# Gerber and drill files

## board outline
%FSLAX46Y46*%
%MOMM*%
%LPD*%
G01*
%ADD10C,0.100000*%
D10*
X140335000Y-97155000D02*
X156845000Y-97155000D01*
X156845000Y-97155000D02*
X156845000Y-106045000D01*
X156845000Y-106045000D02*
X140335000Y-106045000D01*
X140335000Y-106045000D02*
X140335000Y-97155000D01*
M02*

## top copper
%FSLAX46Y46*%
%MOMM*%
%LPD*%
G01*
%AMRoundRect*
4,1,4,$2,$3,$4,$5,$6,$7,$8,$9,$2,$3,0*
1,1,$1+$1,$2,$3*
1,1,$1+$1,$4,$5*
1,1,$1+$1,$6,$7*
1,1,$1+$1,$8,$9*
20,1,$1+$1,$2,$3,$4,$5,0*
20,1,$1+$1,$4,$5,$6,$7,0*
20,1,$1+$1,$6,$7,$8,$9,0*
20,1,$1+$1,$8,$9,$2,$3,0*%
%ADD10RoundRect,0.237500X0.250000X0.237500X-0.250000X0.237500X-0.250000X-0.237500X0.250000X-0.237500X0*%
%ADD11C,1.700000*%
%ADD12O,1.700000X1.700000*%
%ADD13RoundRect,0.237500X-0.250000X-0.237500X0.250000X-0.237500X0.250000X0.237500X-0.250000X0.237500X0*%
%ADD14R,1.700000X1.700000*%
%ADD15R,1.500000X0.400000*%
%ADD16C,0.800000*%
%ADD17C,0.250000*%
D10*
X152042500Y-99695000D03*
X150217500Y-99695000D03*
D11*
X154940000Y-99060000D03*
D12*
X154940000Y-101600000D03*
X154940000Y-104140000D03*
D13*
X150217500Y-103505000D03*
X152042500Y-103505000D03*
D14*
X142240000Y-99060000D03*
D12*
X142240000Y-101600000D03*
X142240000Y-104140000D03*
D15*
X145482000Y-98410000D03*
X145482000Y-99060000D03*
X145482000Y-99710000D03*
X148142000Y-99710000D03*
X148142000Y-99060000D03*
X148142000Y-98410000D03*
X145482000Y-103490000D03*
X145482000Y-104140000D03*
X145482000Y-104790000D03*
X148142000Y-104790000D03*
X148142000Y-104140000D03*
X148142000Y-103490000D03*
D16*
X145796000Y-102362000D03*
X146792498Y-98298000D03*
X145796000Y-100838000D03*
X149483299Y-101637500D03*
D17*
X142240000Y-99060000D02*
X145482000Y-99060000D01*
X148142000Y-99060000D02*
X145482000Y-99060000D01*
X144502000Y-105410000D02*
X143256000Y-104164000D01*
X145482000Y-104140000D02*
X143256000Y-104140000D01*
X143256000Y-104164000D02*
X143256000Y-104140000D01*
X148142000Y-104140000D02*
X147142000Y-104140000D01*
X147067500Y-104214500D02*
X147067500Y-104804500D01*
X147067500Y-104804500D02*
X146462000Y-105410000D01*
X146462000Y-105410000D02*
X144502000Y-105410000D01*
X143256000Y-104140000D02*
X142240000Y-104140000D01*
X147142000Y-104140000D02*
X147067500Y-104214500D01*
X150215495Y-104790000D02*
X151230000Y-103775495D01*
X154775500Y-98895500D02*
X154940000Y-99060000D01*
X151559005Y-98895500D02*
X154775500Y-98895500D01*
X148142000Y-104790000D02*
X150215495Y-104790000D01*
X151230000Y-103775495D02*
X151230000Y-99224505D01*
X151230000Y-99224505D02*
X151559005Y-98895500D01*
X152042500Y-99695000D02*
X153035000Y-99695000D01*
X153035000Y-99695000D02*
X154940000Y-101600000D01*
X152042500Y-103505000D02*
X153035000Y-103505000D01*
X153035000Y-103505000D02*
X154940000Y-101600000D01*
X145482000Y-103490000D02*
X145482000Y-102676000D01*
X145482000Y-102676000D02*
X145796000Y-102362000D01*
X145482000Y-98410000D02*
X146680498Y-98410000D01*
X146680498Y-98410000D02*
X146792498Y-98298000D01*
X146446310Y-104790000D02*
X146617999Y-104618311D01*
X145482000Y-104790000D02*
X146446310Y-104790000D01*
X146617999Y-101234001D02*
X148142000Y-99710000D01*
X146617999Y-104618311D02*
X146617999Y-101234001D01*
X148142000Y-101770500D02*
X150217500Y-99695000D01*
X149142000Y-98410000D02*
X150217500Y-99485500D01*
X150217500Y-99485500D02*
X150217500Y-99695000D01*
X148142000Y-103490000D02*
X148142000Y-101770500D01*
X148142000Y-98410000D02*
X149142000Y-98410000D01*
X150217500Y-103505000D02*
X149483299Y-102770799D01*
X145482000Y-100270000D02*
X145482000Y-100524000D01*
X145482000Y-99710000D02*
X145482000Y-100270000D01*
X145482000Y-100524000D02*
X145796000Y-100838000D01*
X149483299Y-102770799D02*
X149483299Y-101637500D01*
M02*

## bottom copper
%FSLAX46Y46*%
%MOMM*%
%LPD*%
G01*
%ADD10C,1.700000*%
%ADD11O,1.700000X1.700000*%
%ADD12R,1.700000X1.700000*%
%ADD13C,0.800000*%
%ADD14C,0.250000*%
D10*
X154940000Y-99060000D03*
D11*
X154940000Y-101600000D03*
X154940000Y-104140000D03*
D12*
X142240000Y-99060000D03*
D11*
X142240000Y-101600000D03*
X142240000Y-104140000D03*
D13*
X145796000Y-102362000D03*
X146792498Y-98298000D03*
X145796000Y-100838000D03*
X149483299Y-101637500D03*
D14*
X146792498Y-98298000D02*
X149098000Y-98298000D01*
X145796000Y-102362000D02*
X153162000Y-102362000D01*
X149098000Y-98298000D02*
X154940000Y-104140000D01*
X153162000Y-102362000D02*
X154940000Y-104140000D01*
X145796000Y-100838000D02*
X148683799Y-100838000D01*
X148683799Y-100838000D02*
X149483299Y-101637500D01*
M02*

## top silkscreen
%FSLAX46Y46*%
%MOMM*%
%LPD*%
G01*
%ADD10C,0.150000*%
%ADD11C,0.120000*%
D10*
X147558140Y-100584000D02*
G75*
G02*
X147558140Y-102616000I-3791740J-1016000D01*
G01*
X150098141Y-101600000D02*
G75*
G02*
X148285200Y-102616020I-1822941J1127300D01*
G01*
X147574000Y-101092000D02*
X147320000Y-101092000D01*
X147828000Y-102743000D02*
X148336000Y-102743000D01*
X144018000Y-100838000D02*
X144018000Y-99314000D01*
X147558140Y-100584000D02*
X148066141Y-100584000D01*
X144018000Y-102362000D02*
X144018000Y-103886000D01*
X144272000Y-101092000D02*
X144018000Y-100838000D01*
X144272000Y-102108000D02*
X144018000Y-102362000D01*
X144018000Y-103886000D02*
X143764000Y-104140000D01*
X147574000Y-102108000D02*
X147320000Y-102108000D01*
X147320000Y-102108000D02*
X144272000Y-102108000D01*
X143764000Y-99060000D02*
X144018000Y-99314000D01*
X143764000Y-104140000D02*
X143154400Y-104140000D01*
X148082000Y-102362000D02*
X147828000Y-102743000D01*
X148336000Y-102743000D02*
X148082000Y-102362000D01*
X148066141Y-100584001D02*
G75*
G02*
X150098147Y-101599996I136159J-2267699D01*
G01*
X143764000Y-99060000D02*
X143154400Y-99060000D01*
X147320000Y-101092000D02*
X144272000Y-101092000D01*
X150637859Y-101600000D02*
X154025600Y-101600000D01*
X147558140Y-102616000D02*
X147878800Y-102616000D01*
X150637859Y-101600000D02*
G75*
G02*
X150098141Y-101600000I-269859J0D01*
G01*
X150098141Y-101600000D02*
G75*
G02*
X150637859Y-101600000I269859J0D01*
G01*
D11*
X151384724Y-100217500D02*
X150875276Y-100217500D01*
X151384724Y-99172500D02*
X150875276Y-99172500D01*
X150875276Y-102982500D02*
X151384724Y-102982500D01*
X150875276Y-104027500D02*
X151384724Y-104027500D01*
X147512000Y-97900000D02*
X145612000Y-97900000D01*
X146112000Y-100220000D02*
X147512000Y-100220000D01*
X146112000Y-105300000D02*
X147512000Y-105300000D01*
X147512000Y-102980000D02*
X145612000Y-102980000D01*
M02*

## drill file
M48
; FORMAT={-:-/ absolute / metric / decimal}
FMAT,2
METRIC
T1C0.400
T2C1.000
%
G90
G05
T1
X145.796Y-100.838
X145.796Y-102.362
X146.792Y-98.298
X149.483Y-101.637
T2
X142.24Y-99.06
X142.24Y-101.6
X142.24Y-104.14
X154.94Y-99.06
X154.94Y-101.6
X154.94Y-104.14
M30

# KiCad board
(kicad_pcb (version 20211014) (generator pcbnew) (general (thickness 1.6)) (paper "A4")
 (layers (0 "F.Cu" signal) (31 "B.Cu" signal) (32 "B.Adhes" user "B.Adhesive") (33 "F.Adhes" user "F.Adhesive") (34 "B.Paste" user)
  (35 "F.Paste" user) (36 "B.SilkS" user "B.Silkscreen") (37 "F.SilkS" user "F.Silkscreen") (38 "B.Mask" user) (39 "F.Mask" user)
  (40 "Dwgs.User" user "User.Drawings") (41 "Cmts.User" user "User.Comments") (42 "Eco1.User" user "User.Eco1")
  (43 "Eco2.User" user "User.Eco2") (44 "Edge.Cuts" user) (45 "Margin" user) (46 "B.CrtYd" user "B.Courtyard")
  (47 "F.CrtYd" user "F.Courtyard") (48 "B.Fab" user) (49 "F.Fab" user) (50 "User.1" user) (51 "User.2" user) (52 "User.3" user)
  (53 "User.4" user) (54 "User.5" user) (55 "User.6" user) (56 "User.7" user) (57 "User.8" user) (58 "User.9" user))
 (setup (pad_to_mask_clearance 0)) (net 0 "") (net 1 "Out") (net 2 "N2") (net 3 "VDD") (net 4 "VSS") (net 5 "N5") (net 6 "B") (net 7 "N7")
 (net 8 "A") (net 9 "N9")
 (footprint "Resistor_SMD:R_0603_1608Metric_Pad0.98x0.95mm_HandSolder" (layer "F.Cu") (at 151.13 99.695 180)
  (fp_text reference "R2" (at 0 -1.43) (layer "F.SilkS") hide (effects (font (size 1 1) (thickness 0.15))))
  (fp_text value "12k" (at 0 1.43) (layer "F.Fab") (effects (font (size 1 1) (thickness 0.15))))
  (fp_line (start -0.254724 -0.5225) (end 0.254724 -0.5225) (layer "F.SilkS") (width 0.12))
  (fp_line (start -0.254724 0.5225) (end 0.254724 0.5225) (layer "F.SilkS") (width 0.12))
  (pad "1" smd roundrect (at -0.9125 0 180) (size 0.975 0.95) (layers "F.Cu" "F.Paste" "F.Mask") (roundrect_rratio 0.25) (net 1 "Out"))
  (pad "2" smd roundrect (at 0.9125 0 180) (size 0.975 0.95) (layers "F.Cu" "F.Paste" "F.Mask") (roundrect_rratio 0.25) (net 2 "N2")))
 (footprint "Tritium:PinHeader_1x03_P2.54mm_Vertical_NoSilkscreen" (layer "F.Cu") (at 154.94 99.06)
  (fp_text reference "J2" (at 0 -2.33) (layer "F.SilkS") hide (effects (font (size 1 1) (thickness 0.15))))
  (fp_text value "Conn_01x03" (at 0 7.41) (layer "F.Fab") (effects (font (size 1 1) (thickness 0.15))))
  (pad "1" thru_hole circle (at 0 0) (size 1.7 1.7) (drill 1) (layers *.Cu *.Mask) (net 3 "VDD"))
  (pad "2" thru_hole oval (at 0 2.54) (size 1.7 1.7) (drill 1) (layers *.Cu *.Mask) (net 1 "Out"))
  (pad "3" thru_hole oval (at 0 5.08) (size 1.7 1.7) (drill 1) (layers *.Cu *.Mask) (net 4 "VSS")))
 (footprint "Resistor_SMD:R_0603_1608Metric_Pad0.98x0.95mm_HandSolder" (layer "F.Cu") (at 151.13 103.505)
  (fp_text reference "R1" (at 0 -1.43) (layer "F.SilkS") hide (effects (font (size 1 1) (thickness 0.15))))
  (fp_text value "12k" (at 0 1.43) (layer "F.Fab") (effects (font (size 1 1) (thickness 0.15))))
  (fp_line (start -0.254724 -0.5225) (end 0.254724 -0.5225) (layer "F.SilkS") (width 0.12))
  (fp_line (start -0.254724 0.5225) (end 0.254724 0.5225) (layer "F.SilkS") (width 0.12))
  (pad "1" smd roundrect (at -0.9125 0) (size 0.975 0.95) (layers "F.Cu" "F.Paste" "F.Mask") (roundrect_rratio 0.25) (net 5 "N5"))
  (pad "2" smd roundrect (at 0.9125 0) (size 0.975 0.95) (layers "F.Cu" "F.Paste" "F.Mask") (roundrect_rratio 0.25) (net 1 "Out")))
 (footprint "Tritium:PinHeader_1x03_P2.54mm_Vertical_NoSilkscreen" (layer "F.Cu") (at 142.24 99.06)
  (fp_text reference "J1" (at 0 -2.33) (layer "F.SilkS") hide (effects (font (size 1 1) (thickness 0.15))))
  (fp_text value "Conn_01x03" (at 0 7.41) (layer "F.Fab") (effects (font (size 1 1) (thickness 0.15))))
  (pad "1" thru_hole rect (at 0 0) (size 1.7 1.7) (drill 1) (layers *.Cu *.Mask) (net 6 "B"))
  (pad "2" thru_hole oval (at 0 2.54) (size 1.7 1.7) (drill 1) (layers *.Cu *.Mask) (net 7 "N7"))
  (pad "3" thru_hole oval (at 0 5.08) (size 1.7 1.7) (drill 1) (layers *.Cu *.Mask) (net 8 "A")))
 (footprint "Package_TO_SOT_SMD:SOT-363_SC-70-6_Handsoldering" (layer "F.Cu") (at 146.812 99.06)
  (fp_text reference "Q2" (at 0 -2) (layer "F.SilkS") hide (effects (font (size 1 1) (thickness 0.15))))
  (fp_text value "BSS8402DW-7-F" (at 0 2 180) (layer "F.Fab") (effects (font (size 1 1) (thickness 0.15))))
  (fp_line (start 0.7 -1.16) (end -1.2 -1.16) (layer "F.SilkS") (width 0.12))
  (fp_line (start -0.7 1.16) (end 0.7 1.16) (layer "F.SilkS") (width 0.12))
  (pad "1" smd rect (at -1.33 -0.65) (size 1.5 0.4) (layers "F.Cu" "F.Paste" "F.Mask") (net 4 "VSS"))
  (pad "2" smd rect (at -1.33 0) (size 1.5 0.4) (layers "F.Cu" "F.Paste" "F.Mask") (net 6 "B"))
  (pad "3" smd rect (at -1.33 0.65) (size 1.5 0.4) (layers "F.Cu" "F.Paste" "F.Mask") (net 5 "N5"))
  (pad "4" smd rect (at 1.33 0.65) (size 1.5 0.4) (layers "F.Cu" "F.Paste" "F.Mask") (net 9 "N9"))
  (pad "5" smd rect (at 1.33 0) (size 1.5 0.4) (layers "F.Cu" "F.Paste" "F.Mask") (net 6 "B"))
  (pad "6" smd rect (at 1.33 -0.65) (size 1.5 0.4) (layers "F.Cu" "F.Paste" "F.Mask") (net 2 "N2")))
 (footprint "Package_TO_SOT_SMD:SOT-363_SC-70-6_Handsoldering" (layer "F.Cu") (at 146.812 104.14)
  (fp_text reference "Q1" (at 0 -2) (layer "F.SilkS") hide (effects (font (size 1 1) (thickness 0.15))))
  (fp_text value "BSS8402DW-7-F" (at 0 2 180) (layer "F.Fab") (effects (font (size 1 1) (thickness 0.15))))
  (fp_line (start -0.7 1.16) (end 0.7 1.16) (layer "F.SilkS") (width 0.12))
  (fp_line (start 0.7 -1.16) (end -1.2 -1.16) (layer "F.SilkS") (width 0.12))
  (pad "1" smd rect (at -1.33 -0.65) (size 1.5 0.4) (layers "F.Cu" "F.Paste" "F.Mask") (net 4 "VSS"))
  (pad "2" smd rect (at -1.33 0) (size 1.5 0.4) (layers "F.Cu" "F.Paste" "F.Mask") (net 8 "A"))
  (pad "3" smd rect (at -1.33 0.65) (size 1.5 0.4) (layers "F.Cu" "F.Paste" "F.Mask") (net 9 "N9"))
  (pad "4" smd rect (at 1.33 0.65) (size 1.5 0.4) (layers "F.Cu" "F.Paste" "F.Mask") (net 3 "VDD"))
  (pad "5" smd rect (at 1.33 0) (size 1.5 0.4) (layers "F.Cu" "F.Paste" "F.Mask") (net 8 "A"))
  (pad "6" smd rect (at 1.33 -0.65) (size 1.5 0.4) (layers "F.Cu" "F.Paste" "F.Mask") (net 2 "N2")))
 (gr_arc (start 147.55814 100.584) (mid 147.6919 101.6) (end 147.55814 102.616) (layer "F.SilkS") (width 0.15))
 (gr_arc (start 150.098141 101.6) (mid 149.323048 102.342429) (end 148.2852 102.616) (layer "F.SilkS") (width 0.15))
 (gr_line (start 147.574 101.092) (end 147.32 101.092) (layer "F.SilkS") (width 0.15))
 (gr_line (start 147.828 102.743) (end 148.336 102.743) (layer "F.SilkS") (width 0.15))
 (gr_line (start 144.018 100.838) (end 144.018 99.314) (layer "F.SilkS") (width 0.15))
 (gr_line (start 147.55814 100.584) (end 148.066141 100.584) (layer "F.SilkS") (width 0.15))
 (gr_line (start 144.018 102.362) (end 144.018 103.886) (layer "F.SilkS") (width 0.15))
 (gr_line (start 144.272 101.092) (end 144.018 100.838) (layer "F.SilkS") (width 0.15))
 (gr_line (start 144.272 102.108) (end 144.018 102.362) (layer "F.SilkS") (width 0.15))
 (gr_line (start 144.018 103.886) (end 143.764 104.14) (layer "F.SilkS") (width 0.15))
 (gr_line (start 147.574 102.108) (end 147.32 102.108) (layer "F.SilkS") (width 0.15))
 (gr_line (start 147.32 102.108) (end 144.272 102.108) (layer "F.SilkS") (width 0.15))
 (gr_line (start 143.764 99.06) (end 144.018 99.314) (layer "F.SilkS") (width 0.15))
 (gr_line (start 143.764 104.14) (end 143.1544 104.14) (layer "F.SilkS") (width 0.15))
 (gr_line (start 148.082 102.362) (end 147.828 102.743) (layer "F.SilkS") (width 0.15))
 (gr_line (start 148.336 102.743) (end 148.082 102.362) (layer "F.SilkS") (width 0.15))
 (gr_arc (start 148.066141 100.584001) (mid 149.218261 100.819761) (end 150.098141 101.6) (layer "F.SilkS") (width 0.15))
 (gr_line (start 143.764 99.06) (end 143.1544 99.06) (layer "F.SilkS") (width 0.15))
 (gr_line (start 147.32 101.092) (end 144.272 101.092) (layer "F.SilkS") (width 0.15))
 (gr_line (start 150.637859 101.6) (end 154.0256 101.6) (layer "F.SilkS") (width 0.15))
 (gr_line (start 147.55814 102.616) (end 147.8788 102.616) (layer "F.SilkS") (width 0.15))
 (gr_circle (center 150.368 101.6) (end 150.098141 101.6) (layer "F.SilkS") (width 0.15) (fill none))
 (gr_line (start 140.335 97.155) (end 156.845 97.155) (layer "Edge.Cuts") (width 0.1))
 (gr_line (start 156.845 97.155) (end 156.845 106.045) (layer "Edge.Cuts") (width 0.1))
 (gr_line (start 156.845 106.045) (end 140.335 106.045) (layer "Edge.Cuts") (width 0.1))
 (gr_line (start 140.335 106.045) (end 140.335 97.155) (layer "Edge.Cuts") (width 0.1))
 (segment (start 142.24 99.06) (end 145.482 99.06) (width 0.25) (layer "F.Cu") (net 6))
 (segment (start 148.142 99.06) (end 145.482 99.06) (width 0.25) (layer "F.Cu") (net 6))
 (segment (start 144.502 105.41) (end 143.256 104.164) (width 0.25) (layer "F.Cu") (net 8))
 (segment (start 145.482 104.14) (end 143.256 104.14) (width 0.25) (layer "F.Cu") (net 8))
 (segment (start 143.256 104.164) (end 143.256 104.14) (width 0.25) (layer "F.Cu") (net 8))
 (segment (start 148.142 104.14) (end 147.142 104.14) (width 0.25) (layer "F.Cu") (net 8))
 (segment (start 147.0675 104.2145) (end 147.0675 104.8045) (width 0.25) (layer "F.Cu") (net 8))
 (segment (start 147.0675 104.8045) (end 146.462 105.41) (width 0.25) (layer "F.Cu") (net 8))
 (segment (start 146.462 105.41) (end 144.502 105.41) (width 0.25) (layer "F.Cu") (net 8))
 (segment (start 143.256 104.14) (end 142.24 104.14) (width 0.25) (layer "F.Cu") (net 8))
 (segment (start 147.142 104.14) (end 147.0675 104.2145) (width 0.25) (layer "F.Cu") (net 8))
 (segment (start 150.215495 104.79) (end 151.23 103.775495) (width 0.25) (layer "F.Cu") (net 3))
 (segment (start 154.7755 98.8955) (end 154.94 99.06) (width 0.25) (layer "F.Cu") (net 3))
 (segment (start 151.559005 98.8955) (end 154.7755 98.8955) (width 0.25) (layer "F.Cu") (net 3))
 (segment (start 148.142 104.79) (end 150.215495 104.79) (width 0.25) (layer "F.Cu") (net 3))
 (segment (start 151.23 103.775495) (end 151.23 99.224505) (width 0.25) (layer "F.Cu") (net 3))
 (segment (start 151.23 99.224505) (end 151.559005 98.8955) (width 0.25) (layer "F.Cu") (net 3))
 (segment (start 152.0425 99.695) (end 153.035 99.695) (width 0.25) (layer "F.Cu") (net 1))
 (segment (start 153.035 99.695) (end 154.94 101.6) (width 0.25) (layer "F.Cu") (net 1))
 (segment (start 152.0425 103.505) (end 153.035 103.505) (width 0.25) (layer "F.Cu") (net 1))
 (segment (start 153.035 103.505) (end 154.94 101.6) (width 0.25) (layer "F.Cu") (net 1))
 (segment (start 145.482 103.49) (end 145.482 102.676) (width 0.25) (layer "F.Cu") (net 4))
 (segment (start 145.482 102.676) (end 145.796 102.362) (width 0.25) (layer "F.Cu") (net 4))
 (segment (start 145.482 98.41) (end 146.680498 98.41) (width 0.25) (layer "F.Cu") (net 4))
 (segment (start 146.680498 98.41) (end 146.792498 98.298) (width 0.25) (layer "F.Cu") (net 4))
 (via (at 145.796 102.362) (size 0.8) (drill 0.4) (layers "F.Cu" "B.Cu") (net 4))
 (via (at 146.792498 98.298) (size 0.8) (drill 0.4) (layers "F.Cu" "B.Cu") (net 4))
 (segment (start 146.792498 98.298) (end 149.098 98.298) (width 0.25) (layer "B.Cu") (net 4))
 (segment (start 145.796 102.362) (end 153.162 102.362) (width 0.25) (layer "B.Cu") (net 4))
 (segment (start 149.098 98.298) (end 154.94 104.14) (width 0.25) (layer "B.Cu") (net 4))
 (segment (start 153.162 102.362) (end 154.94 104.14) (width 0.25) (layer "B.Cu") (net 4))
 (segment (start 146.44631 104.79) (end 146.617999 104.618311) (width 0.25) (layer "F.Cu") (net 9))
 (segment (start 145.482 104.79) (end 146.44631 104.79) (width 0.25) (layer "F.Cu") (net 9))
 (segment (start 146.617999 101.234001) (end 148.142 99.71) (width 0.25) (layer "F.Cu") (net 9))
 (segment (start 146.617999 104.618311) (end 146.617999 101.234001) (width 0.25) (layer "F.Cu") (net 9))
 (segment (start 148.142 101.7705) (end 150.2175 99.695) (width 0.25) (layer "F.Cu") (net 2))
 (segment (start 149.142 98.41) (end 150.2175 99.4855) (width 0.25) (layer "F.Cu") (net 2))
 (segment (start 150.2175 99.4855) (end 150.2175 99.695) (width 0.25) (layer "F.Cu") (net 2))
 (segment (start 148.142 103.49) (end 148.142 101.7705) (width 0.25) (layer "F.Cu") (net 2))
 (segment (start 148.142 98.41) (end 149.142 98.41) (width 0.25) (layer "F.Cu") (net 2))
 (segment (start 150.2175 103.505) (end 149.483299 102.770799) (width 0.25) (layer "F.Cu") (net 5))
 (segment (start 145.482 100.27) (end 145.482 100.524) (width 0.25) (layer "F.Cu") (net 5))
 (segment (start 145.482 99.71) (end 145.482 100.27) (width 0.25) (layer "F.Cu") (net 5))
 (segment (start 145.482 100.524) (end 145.796 100.838) (width 0.25) (layer "F.Cu") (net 5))
 (segment (start 149.483299 102.770799) (end 149.483299 101.6375) (width 0.25) (layer "F.Cu") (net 5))
 (via (at 145.796 100.838) (size 0.8) (drill 0.4) (layers "F.Cu" "B.Cu") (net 5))
 (via (at 149.483299 101.6375) (size 0.8) (drill 0.4) (layers "F.Cu" "B.Cu") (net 5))
 (segment (start 145.796 100.838) (end 148.683799 100.838) (width 0.25) (layer "B.Cu") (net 5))
 (segment (start 148.683799 100.838) (end 149.483299 101.6375) (width 0.25) (layer "B.Cu") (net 5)))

